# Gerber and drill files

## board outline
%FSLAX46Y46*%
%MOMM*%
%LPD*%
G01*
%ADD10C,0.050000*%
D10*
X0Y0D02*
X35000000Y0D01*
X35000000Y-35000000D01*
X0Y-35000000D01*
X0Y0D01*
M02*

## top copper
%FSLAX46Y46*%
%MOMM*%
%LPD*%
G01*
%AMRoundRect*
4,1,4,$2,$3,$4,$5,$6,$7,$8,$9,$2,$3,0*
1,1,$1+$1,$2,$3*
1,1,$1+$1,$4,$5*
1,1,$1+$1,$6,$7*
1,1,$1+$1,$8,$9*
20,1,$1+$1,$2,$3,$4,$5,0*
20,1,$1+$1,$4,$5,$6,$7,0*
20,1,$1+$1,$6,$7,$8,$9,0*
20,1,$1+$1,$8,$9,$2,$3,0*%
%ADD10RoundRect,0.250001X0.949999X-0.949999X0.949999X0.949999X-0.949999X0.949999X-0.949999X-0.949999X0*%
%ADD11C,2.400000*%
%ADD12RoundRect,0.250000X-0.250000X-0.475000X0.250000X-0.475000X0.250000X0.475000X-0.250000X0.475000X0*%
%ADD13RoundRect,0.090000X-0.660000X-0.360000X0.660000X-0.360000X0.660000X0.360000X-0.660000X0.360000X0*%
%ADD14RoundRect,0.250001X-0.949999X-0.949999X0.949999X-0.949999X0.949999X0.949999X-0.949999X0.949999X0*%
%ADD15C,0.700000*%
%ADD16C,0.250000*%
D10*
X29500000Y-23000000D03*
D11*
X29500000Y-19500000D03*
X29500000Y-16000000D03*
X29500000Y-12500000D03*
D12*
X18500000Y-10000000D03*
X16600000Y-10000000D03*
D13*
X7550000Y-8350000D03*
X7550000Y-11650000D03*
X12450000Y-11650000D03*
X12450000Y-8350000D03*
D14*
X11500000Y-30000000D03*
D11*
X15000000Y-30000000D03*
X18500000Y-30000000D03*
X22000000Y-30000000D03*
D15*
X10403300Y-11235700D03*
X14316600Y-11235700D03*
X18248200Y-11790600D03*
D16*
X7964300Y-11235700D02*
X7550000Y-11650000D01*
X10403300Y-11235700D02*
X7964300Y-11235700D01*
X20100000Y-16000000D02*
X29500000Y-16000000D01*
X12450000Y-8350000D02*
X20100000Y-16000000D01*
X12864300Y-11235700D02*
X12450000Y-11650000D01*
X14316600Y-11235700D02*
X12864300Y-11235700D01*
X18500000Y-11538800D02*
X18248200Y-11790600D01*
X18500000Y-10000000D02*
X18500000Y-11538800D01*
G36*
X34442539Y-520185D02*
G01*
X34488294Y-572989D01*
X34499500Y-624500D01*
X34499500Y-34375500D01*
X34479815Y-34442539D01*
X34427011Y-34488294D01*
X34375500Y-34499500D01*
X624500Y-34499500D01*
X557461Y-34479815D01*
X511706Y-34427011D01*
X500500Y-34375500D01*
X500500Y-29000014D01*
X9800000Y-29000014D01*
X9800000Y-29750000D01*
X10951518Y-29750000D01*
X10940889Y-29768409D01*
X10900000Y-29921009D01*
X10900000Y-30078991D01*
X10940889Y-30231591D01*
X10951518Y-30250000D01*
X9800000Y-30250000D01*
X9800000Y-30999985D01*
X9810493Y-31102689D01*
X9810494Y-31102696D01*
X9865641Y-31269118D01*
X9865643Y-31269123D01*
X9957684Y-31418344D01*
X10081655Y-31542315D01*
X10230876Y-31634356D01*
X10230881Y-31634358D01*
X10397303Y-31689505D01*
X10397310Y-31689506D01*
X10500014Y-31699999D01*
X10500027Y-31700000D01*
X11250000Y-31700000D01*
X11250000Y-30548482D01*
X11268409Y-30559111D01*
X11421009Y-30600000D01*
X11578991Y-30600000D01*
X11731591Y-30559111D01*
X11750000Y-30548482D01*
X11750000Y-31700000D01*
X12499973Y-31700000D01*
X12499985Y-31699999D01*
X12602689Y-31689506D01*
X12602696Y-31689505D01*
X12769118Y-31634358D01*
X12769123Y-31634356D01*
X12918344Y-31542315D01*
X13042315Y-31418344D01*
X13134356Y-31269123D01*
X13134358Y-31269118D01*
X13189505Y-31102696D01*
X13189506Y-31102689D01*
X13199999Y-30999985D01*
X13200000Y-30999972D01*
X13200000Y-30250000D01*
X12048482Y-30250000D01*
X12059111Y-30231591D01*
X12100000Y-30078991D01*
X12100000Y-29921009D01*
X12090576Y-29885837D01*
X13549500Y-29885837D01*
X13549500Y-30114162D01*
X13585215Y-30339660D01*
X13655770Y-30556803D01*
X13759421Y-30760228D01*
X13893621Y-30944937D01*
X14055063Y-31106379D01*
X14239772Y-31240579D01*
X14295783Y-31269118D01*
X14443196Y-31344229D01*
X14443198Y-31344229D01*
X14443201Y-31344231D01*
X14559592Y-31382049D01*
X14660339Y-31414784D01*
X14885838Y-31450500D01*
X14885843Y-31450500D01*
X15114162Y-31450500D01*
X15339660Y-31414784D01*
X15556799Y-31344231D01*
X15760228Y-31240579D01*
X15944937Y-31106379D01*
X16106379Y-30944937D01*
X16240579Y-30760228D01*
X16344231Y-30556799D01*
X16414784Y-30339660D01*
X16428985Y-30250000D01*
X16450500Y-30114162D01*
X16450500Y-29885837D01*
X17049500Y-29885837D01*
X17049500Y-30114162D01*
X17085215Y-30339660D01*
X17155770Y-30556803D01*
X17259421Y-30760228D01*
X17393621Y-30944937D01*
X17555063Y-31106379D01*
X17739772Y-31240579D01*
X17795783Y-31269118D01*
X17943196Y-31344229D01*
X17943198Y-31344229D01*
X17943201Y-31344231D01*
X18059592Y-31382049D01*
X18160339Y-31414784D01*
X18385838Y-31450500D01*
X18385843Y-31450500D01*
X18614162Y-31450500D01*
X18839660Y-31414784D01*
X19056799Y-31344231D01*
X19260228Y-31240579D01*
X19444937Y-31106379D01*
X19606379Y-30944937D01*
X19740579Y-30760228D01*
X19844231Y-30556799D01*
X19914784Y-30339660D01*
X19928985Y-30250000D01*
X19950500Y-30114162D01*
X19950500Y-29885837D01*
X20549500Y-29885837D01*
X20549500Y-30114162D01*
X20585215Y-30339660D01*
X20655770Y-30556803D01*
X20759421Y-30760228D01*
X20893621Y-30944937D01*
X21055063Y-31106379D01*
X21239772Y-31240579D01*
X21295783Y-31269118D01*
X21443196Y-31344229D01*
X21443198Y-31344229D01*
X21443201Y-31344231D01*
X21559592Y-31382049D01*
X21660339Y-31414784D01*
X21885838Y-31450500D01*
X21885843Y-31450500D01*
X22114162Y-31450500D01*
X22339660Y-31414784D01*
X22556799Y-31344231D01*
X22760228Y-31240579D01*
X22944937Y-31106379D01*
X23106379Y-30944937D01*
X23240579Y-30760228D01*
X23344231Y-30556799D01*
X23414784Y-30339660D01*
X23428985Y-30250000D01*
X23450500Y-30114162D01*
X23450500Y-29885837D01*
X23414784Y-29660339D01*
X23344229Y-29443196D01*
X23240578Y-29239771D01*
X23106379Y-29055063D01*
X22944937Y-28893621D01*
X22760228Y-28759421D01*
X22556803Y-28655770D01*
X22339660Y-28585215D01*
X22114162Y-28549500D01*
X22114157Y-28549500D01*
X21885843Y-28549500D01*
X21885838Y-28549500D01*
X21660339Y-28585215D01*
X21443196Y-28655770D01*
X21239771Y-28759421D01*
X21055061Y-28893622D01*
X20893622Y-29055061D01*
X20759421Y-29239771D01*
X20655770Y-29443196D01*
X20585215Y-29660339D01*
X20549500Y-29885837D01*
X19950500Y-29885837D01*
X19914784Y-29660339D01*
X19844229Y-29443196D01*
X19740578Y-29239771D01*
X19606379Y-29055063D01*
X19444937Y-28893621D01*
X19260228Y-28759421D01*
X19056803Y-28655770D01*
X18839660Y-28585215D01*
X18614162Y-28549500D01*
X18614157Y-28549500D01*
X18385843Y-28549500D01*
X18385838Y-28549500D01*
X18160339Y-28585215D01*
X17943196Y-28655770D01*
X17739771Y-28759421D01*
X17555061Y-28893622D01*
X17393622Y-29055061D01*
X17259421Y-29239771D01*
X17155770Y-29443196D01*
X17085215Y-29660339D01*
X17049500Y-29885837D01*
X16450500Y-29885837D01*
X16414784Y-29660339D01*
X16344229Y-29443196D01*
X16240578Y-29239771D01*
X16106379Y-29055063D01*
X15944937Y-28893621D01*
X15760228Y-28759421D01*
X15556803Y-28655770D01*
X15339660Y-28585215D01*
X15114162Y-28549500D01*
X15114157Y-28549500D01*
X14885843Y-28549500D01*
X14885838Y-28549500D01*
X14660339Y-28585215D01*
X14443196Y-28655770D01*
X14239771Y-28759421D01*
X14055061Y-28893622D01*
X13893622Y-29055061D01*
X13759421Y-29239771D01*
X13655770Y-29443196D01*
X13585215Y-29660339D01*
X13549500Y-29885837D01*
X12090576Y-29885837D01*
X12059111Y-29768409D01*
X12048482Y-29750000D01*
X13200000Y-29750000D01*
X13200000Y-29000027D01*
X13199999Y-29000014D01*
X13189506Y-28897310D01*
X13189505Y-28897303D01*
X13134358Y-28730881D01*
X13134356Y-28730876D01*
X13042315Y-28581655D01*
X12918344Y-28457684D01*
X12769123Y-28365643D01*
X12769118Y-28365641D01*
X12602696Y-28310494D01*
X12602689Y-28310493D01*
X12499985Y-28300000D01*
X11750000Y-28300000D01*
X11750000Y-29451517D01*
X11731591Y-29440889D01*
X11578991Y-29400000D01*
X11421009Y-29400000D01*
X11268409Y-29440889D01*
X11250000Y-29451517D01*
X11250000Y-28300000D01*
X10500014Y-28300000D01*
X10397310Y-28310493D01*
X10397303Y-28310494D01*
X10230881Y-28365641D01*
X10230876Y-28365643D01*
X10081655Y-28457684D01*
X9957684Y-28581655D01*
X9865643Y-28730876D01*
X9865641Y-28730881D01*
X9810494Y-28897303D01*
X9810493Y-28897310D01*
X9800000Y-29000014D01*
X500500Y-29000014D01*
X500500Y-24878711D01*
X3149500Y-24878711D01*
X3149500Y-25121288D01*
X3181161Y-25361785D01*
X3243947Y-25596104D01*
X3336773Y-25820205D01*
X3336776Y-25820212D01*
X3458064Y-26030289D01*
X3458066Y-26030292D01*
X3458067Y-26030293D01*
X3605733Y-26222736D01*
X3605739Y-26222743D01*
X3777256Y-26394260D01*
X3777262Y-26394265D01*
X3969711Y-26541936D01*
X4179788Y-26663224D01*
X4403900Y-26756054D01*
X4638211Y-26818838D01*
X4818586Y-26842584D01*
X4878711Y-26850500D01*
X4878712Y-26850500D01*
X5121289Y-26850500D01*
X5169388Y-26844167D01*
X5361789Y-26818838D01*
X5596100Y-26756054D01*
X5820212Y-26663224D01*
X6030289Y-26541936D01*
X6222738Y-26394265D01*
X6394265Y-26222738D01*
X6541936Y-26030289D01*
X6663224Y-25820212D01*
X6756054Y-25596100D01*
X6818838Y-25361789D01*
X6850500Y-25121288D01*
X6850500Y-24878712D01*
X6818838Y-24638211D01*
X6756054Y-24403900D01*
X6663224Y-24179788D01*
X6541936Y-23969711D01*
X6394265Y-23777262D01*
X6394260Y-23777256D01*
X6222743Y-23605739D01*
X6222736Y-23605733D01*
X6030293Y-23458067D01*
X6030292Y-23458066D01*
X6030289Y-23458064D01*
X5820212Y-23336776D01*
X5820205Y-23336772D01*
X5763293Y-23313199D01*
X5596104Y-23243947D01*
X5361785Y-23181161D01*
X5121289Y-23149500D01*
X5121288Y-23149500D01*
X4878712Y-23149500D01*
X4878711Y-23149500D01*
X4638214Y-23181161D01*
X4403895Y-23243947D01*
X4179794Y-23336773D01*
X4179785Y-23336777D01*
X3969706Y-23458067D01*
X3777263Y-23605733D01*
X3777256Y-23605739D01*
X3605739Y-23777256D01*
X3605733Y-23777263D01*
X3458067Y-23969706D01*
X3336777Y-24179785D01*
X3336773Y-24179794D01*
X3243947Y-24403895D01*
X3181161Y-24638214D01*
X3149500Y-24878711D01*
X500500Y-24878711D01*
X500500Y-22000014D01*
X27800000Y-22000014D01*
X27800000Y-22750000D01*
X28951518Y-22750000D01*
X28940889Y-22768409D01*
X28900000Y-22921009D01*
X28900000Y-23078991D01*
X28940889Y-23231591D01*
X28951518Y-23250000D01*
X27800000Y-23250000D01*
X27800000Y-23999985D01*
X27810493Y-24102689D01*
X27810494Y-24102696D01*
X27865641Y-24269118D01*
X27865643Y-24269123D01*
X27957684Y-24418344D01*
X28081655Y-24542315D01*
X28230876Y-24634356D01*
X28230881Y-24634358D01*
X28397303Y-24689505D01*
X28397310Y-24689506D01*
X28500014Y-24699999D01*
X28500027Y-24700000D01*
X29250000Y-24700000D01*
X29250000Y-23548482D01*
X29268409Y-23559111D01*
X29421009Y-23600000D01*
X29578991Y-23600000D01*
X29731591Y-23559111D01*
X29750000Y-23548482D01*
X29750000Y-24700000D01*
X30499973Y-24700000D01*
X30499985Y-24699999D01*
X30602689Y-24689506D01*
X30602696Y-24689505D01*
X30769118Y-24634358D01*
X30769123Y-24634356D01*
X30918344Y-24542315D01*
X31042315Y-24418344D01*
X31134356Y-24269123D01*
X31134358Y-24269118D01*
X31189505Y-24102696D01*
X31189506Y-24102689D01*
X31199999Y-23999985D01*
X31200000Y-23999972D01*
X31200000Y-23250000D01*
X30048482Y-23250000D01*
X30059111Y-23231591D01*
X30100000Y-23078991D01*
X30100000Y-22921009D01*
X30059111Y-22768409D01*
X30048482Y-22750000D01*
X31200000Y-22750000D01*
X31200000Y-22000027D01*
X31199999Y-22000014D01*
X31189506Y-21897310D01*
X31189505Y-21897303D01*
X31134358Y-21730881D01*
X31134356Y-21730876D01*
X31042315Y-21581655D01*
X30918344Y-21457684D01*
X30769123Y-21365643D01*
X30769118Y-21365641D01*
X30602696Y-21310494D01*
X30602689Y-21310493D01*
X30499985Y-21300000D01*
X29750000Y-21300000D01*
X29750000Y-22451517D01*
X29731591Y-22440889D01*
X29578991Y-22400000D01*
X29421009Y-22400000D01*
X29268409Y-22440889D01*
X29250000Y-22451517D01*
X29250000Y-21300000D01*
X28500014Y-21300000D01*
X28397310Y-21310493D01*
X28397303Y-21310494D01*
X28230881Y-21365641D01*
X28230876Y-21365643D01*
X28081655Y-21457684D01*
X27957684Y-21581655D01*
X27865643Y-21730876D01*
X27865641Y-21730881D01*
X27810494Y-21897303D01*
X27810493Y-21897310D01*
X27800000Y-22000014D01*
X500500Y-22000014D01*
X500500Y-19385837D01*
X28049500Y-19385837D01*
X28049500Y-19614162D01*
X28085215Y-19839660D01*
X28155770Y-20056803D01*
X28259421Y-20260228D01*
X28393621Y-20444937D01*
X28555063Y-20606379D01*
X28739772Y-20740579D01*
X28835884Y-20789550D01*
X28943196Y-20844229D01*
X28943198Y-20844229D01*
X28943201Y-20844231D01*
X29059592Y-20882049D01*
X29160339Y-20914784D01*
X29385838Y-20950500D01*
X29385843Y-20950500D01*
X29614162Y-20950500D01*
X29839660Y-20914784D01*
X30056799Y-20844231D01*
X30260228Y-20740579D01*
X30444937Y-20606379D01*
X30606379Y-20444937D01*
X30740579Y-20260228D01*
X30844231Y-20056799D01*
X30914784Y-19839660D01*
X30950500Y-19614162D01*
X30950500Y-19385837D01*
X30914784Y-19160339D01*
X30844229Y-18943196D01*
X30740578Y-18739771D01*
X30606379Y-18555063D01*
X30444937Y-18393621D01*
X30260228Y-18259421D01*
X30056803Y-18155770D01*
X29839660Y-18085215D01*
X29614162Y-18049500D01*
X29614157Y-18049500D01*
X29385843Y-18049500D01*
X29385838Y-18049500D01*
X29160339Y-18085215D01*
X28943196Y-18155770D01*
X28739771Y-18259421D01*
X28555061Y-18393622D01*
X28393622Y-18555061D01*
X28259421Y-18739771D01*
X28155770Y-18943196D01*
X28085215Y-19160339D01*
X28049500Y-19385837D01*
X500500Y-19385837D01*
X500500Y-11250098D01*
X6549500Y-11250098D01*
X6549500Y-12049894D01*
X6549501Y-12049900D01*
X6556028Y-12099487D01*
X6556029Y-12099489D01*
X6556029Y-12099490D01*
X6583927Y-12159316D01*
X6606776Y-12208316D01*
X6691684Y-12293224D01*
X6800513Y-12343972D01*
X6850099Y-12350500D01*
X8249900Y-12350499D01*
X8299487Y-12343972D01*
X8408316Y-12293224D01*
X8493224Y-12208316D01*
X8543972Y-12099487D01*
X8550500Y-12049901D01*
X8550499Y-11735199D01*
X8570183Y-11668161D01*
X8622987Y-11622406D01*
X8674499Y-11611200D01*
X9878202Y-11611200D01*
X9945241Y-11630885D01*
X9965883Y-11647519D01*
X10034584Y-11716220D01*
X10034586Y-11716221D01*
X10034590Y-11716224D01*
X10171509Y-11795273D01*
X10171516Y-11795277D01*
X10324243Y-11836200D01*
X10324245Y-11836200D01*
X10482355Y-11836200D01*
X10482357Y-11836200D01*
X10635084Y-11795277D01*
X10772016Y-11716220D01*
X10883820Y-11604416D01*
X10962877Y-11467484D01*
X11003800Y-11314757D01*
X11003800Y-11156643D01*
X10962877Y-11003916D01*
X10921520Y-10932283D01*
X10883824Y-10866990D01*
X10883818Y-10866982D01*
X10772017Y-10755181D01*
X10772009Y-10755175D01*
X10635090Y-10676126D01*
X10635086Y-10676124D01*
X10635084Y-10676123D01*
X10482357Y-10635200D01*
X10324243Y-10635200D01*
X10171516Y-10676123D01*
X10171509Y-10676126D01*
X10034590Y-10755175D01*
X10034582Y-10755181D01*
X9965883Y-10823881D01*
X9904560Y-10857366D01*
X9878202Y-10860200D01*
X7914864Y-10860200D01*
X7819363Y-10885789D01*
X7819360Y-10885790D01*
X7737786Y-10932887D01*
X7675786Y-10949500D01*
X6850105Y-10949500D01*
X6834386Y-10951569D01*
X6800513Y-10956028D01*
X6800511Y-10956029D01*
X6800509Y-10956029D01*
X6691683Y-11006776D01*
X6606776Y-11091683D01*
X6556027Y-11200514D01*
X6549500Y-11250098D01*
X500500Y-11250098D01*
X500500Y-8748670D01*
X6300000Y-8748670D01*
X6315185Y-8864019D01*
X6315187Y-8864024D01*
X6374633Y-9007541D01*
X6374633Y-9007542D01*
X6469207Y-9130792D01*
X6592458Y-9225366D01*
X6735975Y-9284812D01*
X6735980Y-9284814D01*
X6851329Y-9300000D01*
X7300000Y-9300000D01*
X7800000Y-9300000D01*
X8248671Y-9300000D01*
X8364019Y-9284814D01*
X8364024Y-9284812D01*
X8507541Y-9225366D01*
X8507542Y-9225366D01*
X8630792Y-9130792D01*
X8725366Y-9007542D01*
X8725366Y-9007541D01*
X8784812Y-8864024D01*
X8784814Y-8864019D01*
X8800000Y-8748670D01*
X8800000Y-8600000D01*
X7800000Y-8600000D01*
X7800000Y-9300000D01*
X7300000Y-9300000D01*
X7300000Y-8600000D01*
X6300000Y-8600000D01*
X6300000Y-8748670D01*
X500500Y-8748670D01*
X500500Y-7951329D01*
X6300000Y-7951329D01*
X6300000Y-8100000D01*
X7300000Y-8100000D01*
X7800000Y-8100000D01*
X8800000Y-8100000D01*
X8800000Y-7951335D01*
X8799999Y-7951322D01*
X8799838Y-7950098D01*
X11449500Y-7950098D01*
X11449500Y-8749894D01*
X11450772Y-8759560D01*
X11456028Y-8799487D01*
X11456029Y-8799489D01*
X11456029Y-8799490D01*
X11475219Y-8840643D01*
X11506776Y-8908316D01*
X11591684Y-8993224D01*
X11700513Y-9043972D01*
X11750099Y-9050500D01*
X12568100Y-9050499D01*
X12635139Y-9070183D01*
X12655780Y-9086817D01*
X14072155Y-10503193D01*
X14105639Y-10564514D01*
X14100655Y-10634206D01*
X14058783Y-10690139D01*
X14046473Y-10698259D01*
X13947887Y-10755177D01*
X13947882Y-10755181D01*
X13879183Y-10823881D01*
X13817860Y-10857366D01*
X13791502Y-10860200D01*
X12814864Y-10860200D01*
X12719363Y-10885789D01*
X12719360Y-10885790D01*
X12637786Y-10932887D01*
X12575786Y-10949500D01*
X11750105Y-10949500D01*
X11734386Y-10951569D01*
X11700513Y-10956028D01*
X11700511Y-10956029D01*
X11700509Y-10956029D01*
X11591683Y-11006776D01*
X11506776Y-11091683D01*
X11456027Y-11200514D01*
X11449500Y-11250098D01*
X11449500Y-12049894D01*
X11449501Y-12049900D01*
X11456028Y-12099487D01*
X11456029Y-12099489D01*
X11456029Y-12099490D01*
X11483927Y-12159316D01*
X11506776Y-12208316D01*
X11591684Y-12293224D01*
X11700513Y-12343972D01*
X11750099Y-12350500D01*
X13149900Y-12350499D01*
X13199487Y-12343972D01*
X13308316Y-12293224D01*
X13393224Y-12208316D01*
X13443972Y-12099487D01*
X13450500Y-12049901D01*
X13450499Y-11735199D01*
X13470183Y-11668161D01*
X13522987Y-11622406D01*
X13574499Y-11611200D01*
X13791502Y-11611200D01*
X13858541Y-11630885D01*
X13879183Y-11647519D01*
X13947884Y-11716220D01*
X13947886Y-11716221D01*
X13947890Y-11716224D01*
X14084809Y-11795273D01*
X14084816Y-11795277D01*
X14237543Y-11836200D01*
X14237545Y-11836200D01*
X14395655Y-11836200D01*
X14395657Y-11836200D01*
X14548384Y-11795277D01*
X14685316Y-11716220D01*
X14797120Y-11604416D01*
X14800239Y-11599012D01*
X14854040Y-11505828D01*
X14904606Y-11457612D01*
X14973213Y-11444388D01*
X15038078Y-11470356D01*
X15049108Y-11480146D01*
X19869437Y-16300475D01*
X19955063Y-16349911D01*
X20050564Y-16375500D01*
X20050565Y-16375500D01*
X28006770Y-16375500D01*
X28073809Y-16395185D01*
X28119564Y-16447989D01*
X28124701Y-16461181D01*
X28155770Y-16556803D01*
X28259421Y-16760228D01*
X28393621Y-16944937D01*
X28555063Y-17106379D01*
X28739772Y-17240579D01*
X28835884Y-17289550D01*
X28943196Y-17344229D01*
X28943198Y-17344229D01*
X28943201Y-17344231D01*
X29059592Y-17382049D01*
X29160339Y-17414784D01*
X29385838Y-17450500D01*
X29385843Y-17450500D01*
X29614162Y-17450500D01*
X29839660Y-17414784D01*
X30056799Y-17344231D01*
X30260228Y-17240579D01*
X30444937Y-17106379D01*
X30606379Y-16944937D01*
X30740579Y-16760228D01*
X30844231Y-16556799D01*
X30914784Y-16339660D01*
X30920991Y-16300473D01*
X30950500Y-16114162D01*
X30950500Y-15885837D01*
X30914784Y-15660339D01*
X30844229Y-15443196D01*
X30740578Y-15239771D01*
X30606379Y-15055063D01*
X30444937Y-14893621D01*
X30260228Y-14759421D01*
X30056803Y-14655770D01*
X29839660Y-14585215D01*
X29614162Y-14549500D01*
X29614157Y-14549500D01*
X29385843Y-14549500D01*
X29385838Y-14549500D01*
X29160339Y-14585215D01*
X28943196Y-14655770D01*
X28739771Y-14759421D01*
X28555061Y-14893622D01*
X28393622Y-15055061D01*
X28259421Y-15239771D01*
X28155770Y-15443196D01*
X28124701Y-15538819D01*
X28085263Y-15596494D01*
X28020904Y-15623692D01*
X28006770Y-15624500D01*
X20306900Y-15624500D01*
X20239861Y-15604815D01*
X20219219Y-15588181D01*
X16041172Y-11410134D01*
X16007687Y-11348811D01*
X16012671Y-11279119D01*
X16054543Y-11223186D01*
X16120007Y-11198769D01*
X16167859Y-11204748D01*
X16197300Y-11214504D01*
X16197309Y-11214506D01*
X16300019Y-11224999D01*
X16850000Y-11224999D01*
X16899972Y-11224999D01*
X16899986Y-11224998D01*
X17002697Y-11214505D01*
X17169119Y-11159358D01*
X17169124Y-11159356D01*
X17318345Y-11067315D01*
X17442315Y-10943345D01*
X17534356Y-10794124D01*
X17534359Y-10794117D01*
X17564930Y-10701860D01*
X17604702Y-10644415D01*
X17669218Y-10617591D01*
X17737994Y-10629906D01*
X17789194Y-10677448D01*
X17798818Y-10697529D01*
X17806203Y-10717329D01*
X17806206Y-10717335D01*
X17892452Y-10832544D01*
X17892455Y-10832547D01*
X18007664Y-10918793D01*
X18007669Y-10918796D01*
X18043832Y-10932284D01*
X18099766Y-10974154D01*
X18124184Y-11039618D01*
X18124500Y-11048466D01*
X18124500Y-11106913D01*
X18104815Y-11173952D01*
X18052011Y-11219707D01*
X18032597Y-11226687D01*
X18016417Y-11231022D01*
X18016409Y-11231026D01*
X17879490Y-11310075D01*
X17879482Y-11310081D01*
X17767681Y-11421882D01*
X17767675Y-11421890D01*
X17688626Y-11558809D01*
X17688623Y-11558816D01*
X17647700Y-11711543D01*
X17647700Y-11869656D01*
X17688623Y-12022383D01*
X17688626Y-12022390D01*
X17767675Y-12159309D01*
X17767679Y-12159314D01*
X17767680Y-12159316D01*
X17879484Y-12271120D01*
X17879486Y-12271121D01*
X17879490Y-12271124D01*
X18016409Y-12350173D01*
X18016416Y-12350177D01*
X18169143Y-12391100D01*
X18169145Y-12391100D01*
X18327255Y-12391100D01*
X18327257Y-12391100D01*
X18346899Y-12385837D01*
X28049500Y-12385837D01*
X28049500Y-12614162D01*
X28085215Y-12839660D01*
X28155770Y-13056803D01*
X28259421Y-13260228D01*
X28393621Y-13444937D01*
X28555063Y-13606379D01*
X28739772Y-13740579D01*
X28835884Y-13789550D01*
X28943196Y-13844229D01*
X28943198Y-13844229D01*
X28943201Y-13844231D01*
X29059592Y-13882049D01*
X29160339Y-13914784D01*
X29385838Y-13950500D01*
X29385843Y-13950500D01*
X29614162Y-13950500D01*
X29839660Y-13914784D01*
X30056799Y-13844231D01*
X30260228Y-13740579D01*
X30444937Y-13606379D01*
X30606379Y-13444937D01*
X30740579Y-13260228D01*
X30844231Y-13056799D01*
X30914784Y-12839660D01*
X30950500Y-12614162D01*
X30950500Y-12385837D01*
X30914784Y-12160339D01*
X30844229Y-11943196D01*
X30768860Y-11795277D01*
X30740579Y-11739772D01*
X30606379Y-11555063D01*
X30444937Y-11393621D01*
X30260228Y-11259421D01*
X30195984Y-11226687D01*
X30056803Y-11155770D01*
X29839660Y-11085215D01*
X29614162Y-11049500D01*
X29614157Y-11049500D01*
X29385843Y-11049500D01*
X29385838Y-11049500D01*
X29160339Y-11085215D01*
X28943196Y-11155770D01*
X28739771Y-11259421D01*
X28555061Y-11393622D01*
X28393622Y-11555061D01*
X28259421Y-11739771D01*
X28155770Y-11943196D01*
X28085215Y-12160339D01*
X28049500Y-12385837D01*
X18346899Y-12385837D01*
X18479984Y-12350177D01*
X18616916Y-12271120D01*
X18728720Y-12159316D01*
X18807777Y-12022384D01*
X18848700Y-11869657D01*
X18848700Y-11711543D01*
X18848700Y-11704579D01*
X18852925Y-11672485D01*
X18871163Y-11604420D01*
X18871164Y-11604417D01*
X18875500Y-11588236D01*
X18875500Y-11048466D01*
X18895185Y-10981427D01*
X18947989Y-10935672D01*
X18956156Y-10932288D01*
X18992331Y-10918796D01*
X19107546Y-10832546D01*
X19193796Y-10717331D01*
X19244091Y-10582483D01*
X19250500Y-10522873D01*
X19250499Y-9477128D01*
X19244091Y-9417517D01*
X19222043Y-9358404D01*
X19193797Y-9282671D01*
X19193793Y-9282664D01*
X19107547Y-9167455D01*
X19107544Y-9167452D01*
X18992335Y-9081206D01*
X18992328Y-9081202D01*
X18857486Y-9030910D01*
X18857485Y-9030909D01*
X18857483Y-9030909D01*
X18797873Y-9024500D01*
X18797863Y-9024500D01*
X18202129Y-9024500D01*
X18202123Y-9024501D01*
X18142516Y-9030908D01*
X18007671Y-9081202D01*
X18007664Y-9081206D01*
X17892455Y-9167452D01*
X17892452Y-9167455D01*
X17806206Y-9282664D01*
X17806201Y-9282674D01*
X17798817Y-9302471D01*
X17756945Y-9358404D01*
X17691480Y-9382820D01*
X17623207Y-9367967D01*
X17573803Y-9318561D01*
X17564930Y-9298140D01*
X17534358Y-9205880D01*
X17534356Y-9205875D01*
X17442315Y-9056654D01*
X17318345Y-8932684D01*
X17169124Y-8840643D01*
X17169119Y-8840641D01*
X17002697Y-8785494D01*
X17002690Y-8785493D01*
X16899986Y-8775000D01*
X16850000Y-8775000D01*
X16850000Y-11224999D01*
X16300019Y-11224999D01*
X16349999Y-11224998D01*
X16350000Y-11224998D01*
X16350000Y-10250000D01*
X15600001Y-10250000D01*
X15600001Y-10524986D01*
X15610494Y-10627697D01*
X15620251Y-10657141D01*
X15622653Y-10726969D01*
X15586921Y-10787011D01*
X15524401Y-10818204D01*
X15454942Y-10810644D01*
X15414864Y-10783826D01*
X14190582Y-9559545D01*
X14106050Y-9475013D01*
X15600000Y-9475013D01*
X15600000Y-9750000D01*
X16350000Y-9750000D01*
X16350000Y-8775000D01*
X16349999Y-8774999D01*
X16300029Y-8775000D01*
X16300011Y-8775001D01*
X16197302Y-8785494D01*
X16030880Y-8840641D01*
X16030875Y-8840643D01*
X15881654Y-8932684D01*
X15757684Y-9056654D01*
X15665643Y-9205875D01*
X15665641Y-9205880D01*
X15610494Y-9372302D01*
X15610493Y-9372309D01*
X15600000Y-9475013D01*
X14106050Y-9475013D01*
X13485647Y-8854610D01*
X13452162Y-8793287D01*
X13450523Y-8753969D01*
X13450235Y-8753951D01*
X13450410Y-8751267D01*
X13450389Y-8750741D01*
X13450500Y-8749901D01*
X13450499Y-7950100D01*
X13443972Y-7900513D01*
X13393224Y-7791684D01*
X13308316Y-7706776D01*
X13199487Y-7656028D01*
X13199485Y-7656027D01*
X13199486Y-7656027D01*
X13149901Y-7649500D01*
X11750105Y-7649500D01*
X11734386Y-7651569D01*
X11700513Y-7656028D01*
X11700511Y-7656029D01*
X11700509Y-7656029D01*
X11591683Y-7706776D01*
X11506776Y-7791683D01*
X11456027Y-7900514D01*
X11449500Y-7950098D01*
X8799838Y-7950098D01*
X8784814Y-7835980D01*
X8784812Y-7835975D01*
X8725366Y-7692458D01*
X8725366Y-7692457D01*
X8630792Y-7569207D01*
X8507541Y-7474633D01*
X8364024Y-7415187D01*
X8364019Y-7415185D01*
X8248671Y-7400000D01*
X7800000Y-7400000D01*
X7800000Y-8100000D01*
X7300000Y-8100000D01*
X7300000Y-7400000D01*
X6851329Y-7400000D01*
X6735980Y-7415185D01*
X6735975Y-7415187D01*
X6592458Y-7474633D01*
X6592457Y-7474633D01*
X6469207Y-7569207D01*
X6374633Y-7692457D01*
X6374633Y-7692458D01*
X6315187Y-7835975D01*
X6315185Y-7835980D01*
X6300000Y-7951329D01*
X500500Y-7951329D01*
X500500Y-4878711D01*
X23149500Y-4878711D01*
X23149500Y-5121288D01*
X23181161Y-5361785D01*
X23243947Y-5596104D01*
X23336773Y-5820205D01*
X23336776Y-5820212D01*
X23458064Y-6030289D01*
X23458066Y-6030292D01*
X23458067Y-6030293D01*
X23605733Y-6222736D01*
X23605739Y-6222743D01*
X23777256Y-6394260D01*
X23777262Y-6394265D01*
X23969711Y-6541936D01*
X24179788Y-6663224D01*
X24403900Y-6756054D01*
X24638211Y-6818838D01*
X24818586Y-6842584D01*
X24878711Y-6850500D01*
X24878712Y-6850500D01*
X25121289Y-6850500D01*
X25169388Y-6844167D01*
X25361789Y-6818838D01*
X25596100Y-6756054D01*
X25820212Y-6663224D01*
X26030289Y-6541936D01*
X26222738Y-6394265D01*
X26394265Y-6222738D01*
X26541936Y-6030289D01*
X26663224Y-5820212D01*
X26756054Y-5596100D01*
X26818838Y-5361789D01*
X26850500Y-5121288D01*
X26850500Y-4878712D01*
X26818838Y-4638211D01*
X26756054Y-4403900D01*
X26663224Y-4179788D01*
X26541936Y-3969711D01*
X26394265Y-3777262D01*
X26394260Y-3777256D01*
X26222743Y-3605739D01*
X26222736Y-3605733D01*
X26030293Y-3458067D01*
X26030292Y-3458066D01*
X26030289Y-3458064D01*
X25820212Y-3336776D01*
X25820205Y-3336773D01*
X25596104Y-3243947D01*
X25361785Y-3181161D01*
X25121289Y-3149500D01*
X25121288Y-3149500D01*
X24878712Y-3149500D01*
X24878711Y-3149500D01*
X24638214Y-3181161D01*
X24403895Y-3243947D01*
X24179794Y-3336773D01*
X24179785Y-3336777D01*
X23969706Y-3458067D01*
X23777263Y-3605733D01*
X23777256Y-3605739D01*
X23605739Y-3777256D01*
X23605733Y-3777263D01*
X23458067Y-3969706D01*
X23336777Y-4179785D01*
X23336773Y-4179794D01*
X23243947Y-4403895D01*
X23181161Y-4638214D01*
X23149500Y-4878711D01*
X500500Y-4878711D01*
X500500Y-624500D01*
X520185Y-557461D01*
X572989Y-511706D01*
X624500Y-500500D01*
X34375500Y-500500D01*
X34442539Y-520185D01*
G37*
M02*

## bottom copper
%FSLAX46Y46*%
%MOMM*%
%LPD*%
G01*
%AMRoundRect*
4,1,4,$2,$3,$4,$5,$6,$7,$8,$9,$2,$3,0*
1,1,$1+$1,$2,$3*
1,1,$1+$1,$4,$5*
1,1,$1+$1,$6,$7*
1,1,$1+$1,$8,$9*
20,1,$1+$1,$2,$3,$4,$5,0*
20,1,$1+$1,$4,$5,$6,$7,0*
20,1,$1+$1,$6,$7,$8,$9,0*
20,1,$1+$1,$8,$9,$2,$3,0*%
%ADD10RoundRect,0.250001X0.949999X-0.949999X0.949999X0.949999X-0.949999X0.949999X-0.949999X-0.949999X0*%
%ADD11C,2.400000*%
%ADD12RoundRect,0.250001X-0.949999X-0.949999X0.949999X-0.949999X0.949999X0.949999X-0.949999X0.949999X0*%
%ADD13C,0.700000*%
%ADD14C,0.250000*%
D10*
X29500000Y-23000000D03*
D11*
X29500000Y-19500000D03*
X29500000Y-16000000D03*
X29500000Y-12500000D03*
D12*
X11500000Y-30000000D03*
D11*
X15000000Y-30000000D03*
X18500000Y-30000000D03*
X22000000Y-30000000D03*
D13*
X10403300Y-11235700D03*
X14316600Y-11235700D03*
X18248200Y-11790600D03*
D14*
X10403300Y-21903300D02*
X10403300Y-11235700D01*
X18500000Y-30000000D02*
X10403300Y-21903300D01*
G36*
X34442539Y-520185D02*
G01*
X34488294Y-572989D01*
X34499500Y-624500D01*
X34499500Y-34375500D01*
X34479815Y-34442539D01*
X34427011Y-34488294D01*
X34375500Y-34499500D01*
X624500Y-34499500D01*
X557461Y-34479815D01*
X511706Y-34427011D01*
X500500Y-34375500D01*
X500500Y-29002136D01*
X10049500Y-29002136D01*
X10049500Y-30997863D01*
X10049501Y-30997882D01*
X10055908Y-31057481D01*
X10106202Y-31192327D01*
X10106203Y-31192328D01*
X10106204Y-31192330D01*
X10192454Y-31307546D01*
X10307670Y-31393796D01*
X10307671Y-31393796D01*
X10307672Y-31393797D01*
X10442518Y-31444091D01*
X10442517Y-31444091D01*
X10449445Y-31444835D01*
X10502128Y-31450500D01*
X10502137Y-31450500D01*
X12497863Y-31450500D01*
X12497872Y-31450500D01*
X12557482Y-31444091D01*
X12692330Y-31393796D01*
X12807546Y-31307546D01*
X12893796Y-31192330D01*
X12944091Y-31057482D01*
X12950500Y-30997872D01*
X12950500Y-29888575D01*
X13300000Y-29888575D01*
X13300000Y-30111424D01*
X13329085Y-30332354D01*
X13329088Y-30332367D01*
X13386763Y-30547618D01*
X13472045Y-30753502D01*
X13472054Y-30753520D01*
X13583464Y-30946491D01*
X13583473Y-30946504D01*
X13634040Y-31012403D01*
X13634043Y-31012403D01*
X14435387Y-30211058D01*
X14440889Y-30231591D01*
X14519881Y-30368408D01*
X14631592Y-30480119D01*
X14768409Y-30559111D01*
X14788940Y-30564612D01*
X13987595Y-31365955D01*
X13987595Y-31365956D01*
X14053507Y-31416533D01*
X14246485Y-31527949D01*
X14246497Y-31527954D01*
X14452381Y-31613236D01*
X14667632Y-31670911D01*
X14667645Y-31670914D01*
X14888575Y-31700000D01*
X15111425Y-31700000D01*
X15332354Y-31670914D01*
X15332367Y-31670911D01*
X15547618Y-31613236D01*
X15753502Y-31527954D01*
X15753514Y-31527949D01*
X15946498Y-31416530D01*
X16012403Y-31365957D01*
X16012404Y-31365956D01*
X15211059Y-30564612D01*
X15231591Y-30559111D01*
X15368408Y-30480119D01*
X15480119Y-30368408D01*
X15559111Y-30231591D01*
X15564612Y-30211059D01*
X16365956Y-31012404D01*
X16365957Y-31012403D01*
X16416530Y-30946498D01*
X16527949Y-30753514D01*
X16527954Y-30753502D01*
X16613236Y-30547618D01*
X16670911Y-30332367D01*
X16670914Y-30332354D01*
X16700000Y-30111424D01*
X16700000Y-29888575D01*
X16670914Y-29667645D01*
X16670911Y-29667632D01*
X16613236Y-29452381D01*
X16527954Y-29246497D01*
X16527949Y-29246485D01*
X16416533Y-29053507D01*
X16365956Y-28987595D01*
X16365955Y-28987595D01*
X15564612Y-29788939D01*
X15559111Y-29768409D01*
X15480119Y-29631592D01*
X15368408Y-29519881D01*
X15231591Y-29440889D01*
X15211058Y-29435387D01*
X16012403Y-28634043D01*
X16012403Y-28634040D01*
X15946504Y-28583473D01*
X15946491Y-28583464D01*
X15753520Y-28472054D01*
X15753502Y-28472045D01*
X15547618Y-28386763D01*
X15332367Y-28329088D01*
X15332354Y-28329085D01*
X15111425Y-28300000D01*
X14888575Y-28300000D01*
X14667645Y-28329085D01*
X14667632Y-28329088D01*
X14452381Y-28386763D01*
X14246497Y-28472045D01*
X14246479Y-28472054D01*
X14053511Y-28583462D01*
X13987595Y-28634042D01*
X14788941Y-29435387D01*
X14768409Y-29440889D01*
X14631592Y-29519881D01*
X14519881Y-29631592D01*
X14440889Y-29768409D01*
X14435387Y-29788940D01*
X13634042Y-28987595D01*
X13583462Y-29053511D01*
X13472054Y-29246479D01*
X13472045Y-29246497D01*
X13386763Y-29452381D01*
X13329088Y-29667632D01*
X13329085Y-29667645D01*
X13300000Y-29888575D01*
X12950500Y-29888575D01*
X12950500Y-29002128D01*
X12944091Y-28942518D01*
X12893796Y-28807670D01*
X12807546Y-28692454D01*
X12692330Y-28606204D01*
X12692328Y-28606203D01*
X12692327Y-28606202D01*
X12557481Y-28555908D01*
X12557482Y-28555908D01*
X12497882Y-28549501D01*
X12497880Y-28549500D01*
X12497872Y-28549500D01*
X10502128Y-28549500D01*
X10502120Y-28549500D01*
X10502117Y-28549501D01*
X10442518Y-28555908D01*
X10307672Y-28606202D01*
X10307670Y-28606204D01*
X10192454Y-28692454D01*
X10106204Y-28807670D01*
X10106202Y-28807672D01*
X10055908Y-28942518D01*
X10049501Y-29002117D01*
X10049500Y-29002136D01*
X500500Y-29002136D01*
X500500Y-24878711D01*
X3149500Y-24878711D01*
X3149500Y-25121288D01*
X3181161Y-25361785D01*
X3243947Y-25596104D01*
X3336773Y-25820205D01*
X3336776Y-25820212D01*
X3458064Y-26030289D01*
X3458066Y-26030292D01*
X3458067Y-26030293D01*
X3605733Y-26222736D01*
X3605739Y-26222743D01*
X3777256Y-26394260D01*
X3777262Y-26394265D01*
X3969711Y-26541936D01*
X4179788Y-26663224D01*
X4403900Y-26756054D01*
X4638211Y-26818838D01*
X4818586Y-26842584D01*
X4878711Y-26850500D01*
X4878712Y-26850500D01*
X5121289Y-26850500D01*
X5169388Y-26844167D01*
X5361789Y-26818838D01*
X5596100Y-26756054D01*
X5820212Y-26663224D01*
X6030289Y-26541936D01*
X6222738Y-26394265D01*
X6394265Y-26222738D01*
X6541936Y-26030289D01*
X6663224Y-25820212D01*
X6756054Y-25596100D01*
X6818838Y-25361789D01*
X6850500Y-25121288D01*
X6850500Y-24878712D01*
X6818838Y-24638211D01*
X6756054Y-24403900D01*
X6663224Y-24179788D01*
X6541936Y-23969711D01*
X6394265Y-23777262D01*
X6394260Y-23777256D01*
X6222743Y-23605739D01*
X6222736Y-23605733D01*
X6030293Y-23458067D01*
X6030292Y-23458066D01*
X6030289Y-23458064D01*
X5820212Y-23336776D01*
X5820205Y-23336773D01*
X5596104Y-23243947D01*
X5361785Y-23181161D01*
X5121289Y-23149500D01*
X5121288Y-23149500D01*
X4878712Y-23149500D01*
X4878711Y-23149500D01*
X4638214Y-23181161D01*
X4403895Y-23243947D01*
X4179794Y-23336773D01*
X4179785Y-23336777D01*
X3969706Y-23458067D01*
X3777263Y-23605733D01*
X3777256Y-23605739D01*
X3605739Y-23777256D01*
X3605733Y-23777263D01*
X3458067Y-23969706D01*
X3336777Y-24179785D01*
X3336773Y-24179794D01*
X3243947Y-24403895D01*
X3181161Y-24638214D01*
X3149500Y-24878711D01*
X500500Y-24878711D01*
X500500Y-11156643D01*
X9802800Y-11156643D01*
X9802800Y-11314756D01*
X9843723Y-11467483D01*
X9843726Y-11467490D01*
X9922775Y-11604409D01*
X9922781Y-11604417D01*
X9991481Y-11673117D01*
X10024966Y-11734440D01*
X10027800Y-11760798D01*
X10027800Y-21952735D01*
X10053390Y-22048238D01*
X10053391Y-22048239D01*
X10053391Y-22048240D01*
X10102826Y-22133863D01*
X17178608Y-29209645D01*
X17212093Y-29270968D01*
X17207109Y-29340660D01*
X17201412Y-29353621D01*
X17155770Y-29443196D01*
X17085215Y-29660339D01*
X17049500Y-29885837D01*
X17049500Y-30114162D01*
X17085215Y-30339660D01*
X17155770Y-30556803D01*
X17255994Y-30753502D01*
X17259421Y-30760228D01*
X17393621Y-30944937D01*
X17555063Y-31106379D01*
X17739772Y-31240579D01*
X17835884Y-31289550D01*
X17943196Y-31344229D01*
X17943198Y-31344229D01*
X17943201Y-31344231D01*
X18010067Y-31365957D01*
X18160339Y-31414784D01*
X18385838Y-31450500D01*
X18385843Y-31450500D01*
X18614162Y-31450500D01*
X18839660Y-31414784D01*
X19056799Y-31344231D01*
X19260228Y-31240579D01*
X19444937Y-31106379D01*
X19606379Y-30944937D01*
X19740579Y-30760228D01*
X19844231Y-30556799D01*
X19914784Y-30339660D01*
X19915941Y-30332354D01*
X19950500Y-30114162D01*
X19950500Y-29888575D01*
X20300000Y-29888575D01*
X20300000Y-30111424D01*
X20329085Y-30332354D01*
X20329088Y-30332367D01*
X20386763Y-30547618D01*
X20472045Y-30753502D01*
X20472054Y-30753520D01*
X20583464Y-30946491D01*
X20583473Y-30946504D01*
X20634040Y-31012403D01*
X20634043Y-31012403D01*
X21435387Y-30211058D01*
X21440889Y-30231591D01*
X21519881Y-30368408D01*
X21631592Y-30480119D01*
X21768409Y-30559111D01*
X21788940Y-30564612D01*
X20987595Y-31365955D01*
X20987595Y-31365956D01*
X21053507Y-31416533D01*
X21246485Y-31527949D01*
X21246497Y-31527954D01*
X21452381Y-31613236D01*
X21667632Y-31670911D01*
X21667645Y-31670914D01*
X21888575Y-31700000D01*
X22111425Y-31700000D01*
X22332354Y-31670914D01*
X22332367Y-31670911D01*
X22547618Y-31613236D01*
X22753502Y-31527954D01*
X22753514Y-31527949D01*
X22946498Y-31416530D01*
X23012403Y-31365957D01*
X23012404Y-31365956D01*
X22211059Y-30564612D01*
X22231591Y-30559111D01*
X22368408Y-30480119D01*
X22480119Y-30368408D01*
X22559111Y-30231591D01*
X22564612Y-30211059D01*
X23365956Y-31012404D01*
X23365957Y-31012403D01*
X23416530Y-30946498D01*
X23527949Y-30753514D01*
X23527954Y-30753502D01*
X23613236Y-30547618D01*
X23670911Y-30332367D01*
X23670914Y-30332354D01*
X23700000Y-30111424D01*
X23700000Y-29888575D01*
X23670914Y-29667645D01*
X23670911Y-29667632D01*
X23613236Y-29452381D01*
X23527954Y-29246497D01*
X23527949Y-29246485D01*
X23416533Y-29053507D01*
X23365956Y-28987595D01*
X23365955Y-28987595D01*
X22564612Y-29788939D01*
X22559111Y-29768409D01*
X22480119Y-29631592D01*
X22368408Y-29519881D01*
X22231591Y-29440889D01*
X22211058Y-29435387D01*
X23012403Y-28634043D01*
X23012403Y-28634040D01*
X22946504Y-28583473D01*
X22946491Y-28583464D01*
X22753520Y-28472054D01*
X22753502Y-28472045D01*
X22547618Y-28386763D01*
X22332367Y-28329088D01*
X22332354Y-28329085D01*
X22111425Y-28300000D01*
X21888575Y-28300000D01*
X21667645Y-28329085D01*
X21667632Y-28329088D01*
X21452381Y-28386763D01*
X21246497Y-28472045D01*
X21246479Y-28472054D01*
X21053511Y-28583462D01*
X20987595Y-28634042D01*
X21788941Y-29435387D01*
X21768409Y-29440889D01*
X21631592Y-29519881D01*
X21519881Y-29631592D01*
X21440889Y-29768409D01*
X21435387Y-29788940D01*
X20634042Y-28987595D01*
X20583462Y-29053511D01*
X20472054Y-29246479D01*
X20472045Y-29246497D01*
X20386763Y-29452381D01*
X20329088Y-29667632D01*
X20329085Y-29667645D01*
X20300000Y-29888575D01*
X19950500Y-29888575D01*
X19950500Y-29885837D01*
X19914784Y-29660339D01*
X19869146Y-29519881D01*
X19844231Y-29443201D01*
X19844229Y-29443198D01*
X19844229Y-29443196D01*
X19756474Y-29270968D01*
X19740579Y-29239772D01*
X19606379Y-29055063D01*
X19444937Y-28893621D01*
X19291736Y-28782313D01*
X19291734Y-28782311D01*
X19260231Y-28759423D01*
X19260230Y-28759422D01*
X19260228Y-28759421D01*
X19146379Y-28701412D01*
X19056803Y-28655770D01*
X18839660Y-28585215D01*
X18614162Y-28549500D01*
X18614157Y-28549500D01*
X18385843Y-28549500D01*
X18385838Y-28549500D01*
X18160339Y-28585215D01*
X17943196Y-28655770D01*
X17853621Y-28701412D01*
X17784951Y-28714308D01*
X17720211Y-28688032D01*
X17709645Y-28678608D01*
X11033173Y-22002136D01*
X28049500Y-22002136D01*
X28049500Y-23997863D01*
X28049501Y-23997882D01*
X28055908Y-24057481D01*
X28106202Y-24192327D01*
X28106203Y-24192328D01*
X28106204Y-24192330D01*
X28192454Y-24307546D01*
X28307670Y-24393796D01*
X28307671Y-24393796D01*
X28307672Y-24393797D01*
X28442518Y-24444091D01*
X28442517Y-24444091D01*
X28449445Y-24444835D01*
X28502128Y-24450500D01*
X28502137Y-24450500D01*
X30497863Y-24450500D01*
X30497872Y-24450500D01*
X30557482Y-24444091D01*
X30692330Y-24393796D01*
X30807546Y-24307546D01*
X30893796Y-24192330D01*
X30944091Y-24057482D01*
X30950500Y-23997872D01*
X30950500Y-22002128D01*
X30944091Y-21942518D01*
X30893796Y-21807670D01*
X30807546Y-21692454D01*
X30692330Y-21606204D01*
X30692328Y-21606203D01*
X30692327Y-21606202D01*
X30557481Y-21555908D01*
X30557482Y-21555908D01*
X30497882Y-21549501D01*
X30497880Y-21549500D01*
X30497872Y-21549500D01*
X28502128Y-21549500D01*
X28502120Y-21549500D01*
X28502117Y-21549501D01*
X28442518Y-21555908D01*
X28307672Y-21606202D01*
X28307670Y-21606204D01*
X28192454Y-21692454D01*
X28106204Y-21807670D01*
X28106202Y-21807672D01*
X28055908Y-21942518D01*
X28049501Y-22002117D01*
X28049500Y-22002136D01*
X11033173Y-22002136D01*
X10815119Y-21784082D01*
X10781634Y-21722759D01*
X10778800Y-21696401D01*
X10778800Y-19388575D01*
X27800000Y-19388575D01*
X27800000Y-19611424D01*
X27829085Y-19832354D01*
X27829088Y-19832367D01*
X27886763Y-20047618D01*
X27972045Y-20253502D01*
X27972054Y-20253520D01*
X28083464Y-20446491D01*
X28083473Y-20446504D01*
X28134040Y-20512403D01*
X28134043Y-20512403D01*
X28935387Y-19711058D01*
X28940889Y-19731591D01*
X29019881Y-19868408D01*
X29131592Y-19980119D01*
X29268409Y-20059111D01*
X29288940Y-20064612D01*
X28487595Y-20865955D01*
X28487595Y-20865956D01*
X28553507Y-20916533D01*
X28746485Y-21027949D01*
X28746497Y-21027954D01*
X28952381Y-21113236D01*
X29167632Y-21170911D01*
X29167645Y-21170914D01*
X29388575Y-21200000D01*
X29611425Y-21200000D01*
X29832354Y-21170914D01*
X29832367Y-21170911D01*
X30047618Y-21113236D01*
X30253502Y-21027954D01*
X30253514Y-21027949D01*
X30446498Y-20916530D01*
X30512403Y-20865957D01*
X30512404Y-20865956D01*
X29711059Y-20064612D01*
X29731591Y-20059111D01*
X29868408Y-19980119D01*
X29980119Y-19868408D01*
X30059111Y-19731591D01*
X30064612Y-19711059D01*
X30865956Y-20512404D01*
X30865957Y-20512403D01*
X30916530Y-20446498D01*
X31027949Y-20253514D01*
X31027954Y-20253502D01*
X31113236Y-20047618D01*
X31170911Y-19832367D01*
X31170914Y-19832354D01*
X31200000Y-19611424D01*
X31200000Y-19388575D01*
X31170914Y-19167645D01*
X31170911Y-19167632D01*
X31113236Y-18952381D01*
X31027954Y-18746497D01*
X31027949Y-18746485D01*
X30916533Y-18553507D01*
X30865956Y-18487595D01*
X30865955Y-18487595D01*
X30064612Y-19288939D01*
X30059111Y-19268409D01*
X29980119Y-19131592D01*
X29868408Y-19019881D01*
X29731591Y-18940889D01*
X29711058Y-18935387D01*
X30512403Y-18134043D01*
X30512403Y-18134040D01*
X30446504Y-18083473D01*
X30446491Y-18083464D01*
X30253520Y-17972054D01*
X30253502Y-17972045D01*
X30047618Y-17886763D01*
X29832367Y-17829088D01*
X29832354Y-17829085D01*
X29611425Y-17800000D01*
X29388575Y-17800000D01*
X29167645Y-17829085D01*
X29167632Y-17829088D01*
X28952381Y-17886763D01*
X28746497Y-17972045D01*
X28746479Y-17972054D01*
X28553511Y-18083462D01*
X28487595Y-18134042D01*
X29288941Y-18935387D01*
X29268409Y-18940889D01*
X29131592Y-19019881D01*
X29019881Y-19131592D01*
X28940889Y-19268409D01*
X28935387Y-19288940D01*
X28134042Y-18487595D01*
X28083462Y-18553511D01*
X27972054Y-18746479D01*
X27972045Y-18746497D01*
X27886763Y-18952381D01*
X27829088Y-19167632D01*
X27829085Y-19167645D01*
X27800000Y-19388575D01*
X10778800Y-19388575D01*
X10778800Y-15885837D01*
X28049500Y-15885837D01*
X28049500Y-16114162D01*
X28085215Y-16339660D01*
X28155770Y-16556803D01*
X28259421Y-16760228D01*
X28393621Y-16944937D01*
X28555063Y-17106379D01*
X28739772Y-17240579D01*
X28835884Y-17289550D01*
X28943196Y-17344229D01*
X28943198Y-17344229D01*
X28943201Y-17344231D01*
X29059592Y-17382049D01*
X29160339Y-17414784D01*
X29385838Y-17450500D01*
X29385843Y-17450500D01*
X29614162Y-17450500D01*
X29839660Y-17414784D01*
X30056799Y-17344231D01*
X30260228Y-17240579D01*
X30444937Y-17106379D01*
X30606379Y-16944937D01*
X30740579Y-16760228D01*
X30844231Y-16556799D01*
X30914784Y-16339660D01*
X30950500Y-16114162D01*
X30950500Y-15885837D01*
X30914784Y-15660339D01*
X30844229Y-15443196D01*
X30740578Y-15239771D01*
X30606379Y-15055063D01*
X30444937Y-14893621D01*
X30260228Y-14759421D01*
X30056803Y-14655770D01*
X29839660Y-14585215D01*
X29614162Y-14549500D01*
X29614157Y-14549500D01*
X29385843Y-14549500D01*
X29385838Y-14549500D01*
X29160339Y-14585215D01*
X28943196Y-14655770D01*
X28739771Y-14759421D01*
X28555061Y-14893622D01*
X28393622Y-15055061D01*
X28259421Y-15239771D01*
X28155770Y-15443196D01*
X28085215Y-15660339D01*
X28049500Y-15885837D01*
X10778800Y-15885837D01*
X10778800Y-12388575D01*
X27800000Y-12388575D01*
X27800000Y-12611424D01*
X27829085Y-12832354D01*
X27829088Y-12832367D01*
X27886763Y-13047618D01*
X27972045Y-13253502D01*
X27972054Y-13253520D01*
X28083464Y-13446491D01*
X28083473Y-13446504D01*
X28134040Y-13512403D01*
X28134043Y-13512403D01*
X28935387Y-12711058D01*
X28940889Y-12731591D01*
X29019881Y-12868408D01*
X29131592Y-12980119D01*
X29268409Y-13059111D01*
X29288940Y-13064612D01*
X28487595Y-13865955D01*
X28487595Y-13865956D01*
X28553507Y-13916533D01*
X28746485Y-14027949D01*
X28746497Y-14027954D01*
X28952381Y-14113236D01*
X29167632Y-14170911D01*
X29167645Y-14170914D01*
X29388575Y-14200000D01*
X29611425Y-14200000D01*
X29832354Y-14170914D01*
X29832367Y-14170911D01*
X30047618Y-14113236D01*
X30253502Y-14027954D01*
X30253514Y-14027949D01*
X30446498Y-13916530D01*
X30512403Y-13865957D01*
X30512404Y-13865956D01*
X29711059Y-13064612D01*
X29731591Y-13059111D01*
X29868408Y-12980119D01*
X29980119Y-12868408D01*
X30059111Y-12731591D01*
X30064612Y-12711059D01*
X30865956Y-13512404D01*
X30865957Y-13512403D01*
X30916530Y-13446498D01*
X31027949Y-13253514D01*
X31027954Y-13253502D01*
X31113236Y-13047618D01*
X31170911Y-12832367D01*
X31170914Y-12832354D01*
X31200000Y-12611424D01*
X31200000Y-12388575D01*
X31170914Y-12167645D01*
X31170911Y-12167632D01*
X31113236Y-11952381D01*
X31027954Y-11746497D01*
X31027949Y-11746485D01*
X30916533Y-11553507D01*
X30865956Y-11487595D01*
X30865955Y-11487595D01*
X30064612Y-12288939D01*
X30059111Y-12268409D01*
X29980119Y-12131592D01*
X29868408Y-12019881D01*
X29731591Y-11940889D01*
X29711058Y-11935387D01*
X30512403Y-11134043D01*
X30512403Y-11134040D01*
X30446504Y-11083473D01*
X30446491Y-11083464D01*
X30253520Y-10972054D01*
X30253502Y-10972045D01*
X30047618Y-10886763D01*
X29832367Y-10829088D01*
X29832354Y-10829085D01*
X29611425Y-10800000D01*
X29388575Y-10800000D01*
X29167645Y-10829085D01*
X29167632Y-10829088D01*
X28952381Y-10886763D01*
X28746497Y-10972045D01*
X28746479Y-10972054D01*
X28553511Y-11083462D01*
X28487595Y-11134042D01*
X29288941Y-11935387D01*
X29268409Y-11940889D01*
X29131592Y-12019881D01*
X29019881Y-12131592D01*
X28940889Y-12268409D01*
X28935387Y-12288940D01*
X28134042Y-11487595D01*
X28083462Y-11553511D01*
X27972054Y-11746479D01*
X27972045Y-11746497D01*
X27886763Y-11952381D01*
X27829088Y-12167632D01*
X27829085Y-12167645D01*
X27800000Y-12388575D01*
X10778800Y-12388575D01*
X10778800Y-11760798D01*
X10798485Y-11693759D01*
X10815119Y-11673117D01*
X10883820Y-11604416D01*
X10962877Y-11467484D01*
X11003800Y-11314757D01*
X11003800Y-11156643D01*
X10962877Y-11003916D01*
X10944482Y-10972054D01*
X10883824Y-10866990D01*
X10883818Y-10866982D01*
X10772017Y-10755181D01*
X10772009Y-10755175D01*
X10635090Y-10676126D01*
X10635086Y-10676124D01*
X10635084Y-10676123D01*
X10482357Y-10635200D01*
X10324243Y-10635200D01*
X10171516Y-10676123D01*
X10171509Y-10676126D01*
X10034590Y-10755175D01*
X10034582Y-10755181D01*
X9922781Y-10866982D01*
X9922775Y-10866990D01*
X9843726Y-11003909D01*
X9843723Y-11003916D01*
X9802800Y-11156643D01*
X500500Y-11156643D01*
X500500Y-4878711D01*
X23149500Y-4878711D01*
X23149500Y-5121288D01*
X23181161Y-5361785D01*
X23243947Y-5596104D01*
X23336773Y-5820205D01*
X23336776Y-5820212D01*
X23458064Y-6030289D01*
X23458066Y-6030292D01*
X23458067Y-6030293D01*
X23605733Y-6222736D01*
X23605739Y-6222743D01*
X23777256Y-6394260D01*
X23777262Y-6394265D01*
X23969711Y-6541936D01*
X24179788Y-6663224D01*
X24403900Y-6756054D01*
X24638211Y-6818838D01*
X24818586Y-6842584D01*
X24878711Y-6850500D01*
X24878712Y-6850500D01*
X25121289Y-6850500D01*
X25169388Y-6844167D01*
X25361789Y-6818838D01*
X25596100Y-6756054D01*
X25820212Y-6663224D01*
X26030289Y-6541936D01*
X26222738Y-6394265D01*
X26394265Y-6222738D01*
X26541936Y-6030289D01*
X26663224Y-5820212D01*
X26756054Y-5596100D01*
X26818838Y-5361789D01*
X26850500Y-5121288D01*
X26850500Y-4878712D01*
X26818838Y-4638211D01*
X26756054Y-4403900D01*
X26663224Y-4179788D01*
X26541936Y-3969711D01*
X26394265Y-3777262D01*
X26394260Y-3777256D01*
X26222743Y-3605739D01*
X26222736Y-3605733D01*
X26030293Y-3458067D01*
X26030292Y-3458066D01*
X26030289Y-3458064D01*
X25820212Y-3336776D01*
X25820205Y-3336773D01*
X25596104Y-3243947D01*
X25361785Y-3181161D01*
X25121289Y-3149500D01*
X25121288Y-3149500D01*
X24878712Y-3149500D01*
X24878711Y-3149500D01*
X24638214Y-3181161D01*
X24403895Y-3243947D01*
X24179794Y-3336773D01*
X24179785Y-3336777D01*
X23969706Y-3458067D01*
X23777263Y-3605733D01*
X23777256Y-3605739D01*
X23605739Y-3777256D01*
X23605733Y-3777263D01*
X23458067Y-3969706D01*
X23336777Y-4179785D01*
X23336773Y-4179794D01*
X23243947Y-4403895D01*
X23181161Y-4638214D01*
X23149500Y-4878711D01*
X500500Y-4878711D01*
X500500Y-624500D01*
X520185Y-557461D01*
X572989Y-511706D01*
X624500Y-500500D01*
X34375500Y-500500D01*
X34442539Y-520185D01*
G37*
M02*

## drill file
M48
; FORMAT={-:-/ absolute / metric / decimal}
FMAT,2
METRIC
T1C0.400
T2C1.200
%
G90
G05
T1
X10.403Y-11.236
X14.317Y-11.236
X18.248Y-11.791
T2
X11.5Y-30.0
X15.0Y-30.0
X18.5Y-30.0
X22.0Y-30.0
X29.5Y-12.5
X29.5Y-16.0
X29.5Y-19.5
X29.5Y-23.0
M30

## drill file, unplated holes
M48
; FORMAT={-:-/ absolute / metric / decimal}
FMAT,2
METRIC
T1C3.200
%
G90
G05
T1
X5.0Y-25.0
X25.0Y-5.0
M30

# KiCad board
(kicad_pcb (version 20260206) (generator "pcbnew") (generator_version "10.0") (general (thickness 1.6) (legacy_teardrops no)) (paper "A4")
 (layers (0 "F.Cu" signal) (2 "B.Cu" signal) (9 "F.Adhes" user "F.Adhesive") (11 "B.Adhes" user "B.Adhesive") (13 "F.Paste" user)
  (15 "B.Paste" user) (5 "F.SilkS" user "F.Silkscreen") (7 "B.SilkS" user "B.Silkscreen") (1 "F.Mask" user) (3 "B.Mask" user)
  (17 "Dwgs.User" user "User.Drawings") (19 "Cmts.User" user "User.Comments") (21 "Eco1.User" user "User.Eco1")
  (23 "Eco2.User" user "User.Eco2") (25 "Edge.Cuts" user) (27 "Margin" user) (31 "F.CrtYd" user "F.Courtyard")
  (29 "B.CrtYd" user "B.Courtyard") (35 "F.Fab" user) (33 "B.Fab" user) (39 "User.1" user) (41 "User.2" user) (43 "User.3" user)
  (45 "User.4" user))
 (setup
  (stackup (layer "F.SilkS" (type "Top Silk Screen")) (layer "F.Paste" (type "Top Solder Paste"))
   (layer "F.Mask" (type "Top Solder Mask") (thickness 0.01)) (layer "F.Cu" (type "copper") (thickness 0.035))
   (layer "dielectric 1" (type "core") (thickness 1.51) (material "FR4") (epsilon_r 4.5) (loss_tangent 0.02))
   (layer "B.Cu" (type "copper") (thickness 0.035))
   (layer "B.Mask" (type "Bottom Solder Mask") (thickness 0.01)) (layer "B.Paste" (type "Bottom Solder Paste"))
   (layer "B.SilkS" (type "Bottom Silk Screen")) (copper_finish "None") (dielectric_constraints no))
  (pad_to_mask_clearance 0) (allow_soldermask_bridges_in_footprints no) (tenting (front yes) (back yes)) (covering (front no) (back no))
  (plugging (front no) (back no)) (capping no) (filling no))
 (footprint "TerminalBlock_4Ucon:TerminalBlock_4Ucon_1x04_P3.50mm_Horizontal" (layer "F.Cu") (at 29.5 23 90)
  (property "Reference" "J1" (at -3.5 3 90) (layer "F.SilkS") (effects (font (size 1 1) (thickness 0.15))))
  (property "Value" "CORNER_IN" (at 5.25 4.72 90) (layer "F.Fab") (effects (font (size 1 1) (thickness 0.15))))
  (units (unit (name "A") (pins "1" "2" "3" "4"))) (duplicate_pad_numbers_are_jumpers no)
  (pad "1" thru_hole roundrect (at 0 0 90) (size 2.4 2.4) (drill 1.2) (layers "*.Cu" "*.Mask") (remove_unused_layers no)
   (roundrect_rratio 0.104167) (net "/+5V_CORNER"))
  (pad "2" thru_hole circle (at 3.5 0 90) (size 2.4 2.4) (drill 1.2) (layers "*.Cu" "*.Mask") (remove_unused_layers no) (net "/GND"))
  (pad "3" thru_hole circle (at 7 0 90) (size 2.4 2.4) (drill 1.2) (layers "*.Cu" "*.Mask") (remove_unused_layers no) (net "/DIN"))
  (pad "4" thru_hole circle (at 10.5 0 90) (size 2.4 2.4) (drill 1.2) (layers "*.Cu" "*.Mask") (remove_unused_layers no) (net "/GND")))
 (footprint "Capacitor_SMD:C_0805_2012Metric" (layer "F.Cu") (at 17.55 10)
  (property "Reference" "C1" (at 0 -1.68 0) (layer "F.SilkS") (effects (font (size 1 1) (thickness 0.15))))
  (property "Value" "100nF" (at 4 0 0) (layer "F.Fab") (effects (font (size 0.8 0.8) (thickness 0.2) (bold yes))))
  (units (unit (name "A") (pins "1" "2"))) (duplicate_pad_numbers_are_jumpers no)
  (pad "1" smd roundrect (at -0.95 0) (size 1 1.45) (layers "F.Cu" "F.Mask" "F.Paste") (roundrect_rratio 0.25) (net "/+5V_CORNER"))
  (pad "2" smd roundrect (at 0.95 0) (size 1 1.45) (layers "F.Cu" "F.Mask" "F.Paste") (roundrect_rratio 0.25) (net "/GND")))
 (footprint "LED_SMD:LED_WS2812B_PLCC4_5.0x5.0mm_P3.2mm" (layer "F.Cu") (at 10 10)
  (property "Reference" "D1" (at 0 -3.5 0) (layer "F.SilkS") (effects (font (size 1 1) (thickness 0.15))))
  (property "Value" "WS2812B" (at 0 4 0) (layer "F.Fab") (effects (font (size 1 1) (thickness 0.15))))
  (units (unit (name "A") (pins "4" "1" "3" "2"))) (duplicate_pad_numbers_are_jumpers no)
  (pad "1" smd roundrect (at -2.45 -1.65) (size 1.5 0.9) (layers "F.Cu" "F.Mask" "F.Paste") (roundrect_rratio 0.1) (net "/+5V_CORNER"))
  (pad "2" smd roundrect (at -2.45 1.65) (size 1.5 0.9) (layers "F.Cu" "F.Mask" "F.Paste") (roundrect_rratio 0.1) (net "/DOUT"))
  (pad "3" smd roundrect (at 2.45 1.65) (size 1.5 0.9) (layers "F.Cu" "F.Mask" "F.Paste") (roundrect_rratio 0.1) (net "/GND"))
  (pad "4" smd roundrect (at 2.45 -1.65) (size 1.5 0.9) (layers "F.Cu" "F.Mask" "F.Paste") (roundrect_rratio 0.1) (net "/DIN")))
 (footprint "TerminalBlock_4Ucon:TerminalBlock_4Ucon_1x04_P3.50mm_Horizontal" (layer "F.Cu") (at 11.5 30)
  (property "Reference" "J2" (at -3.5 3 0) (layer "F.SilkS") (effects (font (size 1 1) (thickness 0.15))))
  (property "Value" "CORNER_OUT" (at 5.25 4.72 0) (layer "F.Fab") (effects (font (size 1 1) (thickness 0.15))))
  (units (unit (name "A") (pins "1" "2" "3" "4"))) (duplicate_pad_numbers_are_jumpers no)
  (pad "1" thru_hole roundrect (at 0 0) (size 2.4 2.4) (drill 1.2) (layers "*.Cu" "*.Mask") (remove_unused_layers no)
   (roundrect_rratio 0.104167) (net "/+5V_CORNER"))
  (pad "2" thru_hole circle (at 3.5 0) (size 2.4 2.4) (drill 1.2) (layers "*.Cu" "*.Mask") (remove_unused_layers no) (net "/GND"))
  (pad "3" thru_hole circle (at 7 0) (size 2.4 2.4) (drill 1.2) (layers "*.Cu" "*.Mask") (remove_unused_layers no) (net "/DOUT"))
  (pad "4" thru_hole circle (at 10.5 0) (size 2.4 2.4) (drill 1.2) (layers "*.Cu" "*.Mask") (remove_unused_layers no) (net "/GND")))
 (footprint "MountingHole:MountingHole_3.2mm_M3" (layer "F.Cu") (at 25 5 90)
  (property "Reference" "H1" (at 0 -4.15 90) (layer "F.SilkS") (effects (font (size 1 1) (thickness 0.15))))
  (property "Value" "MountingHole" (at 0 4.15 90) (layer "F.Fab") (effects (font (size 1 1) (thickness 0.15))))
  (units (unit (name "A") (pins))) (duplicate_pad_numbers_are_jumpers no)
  (pad "" np_thru_hole circle (at 0 0 90) (size 3.2 3.2) (drill 3.2) (layers "*.Cu" "*.Mask")))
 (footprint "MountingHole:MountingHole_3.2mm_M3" (layer "F.Cu") (at 5 25)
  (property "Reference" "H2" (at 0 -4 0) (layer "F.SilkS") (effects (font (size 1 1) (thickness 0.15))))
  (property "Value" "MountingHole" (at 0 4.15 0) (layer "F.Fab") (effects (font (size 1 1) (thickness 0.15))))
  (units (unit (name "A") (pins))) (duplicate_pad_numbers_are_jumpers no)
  (pad "" np_thru_hole circle (at 0 0) (size 3.2 3.2) (drill 3.2) (layers "*.Cu" "*.Mask")))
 (gr_rect (start 0 0) (end 35 35) (stroke (width 0.05) (type default)) (fill no) (layer "Edge.Cuts"))
 (segment (start 18.5 11.5388) (end 18.2482 11.7906) (width 0.25) (layer "F.Cu") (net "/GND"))
 (segment (start 14.3166 11.2357) (end 12.8643 11.2357) (width 0.25) (layer "F.Cu") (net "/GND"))
 (segment (start 18.5 10) (end 18.5 11.5388) (width 0.25) (layer "F.Cu") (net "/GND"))
 (segment (start 12.8643 11.2357) (end 12.45 11.65) (width 0.25) (layer "F.Cu") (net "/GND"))
 (via (at 14.3166 11.2357) (size 0.7) (drill 0.4) (layers "F.Cu" "B.Cu") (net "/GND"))
 (via (at 18.2482 11.7906) (size 0.7) (drill 0.4) (layers "F.Cu" "B.Cu") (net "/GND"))
 (segment (start 20.1 16) (end 29.5 16) (width 0.25) (layer "F.Cu") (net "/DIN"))
 (segment (start 12.45 8.35) (end 20.1 16) (width 0.25) (layer "F.Cu") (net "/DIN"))
 (segment (start 7.9643 11.2357) (end 7.55 11.65) (width 0.25) (layer "F.Cu") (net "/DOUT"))
 (segment (start 10.4033 11.2357) (end 7.9643 11.2357) (width 0.25) (layer "F.Cu") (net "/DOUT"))
 (via (at 10.4033 11.2357) (size 0.7) (drill 0.4) (layers "F.Cu" "B.Cu") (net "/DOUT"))
 (segment (start 10.4033 21.9033) (end 10.4033 11.2357) (width 0.25) (layer "B.Cu") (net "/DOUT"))
 (segment (start 18.5 30) (end 10.4033 21.9033) (width 0.25) (layer "B.Cu") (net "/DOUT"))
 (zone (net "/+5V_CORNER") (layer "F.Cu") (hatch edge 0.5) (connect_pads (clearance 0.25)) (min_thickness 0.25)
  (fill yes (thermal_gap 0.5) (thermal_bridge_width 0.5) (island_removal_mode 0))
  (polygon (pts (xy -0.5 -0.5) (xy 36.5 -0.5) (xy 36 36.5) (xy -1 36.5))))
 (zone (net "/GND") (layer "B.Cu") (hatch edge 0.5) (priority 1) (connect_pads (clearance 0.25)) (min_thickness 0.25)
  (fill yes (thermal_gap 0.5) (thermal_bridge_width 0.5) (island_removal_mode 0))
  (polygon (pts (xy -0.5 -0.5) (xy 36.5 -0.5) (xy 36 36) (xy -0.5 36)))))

